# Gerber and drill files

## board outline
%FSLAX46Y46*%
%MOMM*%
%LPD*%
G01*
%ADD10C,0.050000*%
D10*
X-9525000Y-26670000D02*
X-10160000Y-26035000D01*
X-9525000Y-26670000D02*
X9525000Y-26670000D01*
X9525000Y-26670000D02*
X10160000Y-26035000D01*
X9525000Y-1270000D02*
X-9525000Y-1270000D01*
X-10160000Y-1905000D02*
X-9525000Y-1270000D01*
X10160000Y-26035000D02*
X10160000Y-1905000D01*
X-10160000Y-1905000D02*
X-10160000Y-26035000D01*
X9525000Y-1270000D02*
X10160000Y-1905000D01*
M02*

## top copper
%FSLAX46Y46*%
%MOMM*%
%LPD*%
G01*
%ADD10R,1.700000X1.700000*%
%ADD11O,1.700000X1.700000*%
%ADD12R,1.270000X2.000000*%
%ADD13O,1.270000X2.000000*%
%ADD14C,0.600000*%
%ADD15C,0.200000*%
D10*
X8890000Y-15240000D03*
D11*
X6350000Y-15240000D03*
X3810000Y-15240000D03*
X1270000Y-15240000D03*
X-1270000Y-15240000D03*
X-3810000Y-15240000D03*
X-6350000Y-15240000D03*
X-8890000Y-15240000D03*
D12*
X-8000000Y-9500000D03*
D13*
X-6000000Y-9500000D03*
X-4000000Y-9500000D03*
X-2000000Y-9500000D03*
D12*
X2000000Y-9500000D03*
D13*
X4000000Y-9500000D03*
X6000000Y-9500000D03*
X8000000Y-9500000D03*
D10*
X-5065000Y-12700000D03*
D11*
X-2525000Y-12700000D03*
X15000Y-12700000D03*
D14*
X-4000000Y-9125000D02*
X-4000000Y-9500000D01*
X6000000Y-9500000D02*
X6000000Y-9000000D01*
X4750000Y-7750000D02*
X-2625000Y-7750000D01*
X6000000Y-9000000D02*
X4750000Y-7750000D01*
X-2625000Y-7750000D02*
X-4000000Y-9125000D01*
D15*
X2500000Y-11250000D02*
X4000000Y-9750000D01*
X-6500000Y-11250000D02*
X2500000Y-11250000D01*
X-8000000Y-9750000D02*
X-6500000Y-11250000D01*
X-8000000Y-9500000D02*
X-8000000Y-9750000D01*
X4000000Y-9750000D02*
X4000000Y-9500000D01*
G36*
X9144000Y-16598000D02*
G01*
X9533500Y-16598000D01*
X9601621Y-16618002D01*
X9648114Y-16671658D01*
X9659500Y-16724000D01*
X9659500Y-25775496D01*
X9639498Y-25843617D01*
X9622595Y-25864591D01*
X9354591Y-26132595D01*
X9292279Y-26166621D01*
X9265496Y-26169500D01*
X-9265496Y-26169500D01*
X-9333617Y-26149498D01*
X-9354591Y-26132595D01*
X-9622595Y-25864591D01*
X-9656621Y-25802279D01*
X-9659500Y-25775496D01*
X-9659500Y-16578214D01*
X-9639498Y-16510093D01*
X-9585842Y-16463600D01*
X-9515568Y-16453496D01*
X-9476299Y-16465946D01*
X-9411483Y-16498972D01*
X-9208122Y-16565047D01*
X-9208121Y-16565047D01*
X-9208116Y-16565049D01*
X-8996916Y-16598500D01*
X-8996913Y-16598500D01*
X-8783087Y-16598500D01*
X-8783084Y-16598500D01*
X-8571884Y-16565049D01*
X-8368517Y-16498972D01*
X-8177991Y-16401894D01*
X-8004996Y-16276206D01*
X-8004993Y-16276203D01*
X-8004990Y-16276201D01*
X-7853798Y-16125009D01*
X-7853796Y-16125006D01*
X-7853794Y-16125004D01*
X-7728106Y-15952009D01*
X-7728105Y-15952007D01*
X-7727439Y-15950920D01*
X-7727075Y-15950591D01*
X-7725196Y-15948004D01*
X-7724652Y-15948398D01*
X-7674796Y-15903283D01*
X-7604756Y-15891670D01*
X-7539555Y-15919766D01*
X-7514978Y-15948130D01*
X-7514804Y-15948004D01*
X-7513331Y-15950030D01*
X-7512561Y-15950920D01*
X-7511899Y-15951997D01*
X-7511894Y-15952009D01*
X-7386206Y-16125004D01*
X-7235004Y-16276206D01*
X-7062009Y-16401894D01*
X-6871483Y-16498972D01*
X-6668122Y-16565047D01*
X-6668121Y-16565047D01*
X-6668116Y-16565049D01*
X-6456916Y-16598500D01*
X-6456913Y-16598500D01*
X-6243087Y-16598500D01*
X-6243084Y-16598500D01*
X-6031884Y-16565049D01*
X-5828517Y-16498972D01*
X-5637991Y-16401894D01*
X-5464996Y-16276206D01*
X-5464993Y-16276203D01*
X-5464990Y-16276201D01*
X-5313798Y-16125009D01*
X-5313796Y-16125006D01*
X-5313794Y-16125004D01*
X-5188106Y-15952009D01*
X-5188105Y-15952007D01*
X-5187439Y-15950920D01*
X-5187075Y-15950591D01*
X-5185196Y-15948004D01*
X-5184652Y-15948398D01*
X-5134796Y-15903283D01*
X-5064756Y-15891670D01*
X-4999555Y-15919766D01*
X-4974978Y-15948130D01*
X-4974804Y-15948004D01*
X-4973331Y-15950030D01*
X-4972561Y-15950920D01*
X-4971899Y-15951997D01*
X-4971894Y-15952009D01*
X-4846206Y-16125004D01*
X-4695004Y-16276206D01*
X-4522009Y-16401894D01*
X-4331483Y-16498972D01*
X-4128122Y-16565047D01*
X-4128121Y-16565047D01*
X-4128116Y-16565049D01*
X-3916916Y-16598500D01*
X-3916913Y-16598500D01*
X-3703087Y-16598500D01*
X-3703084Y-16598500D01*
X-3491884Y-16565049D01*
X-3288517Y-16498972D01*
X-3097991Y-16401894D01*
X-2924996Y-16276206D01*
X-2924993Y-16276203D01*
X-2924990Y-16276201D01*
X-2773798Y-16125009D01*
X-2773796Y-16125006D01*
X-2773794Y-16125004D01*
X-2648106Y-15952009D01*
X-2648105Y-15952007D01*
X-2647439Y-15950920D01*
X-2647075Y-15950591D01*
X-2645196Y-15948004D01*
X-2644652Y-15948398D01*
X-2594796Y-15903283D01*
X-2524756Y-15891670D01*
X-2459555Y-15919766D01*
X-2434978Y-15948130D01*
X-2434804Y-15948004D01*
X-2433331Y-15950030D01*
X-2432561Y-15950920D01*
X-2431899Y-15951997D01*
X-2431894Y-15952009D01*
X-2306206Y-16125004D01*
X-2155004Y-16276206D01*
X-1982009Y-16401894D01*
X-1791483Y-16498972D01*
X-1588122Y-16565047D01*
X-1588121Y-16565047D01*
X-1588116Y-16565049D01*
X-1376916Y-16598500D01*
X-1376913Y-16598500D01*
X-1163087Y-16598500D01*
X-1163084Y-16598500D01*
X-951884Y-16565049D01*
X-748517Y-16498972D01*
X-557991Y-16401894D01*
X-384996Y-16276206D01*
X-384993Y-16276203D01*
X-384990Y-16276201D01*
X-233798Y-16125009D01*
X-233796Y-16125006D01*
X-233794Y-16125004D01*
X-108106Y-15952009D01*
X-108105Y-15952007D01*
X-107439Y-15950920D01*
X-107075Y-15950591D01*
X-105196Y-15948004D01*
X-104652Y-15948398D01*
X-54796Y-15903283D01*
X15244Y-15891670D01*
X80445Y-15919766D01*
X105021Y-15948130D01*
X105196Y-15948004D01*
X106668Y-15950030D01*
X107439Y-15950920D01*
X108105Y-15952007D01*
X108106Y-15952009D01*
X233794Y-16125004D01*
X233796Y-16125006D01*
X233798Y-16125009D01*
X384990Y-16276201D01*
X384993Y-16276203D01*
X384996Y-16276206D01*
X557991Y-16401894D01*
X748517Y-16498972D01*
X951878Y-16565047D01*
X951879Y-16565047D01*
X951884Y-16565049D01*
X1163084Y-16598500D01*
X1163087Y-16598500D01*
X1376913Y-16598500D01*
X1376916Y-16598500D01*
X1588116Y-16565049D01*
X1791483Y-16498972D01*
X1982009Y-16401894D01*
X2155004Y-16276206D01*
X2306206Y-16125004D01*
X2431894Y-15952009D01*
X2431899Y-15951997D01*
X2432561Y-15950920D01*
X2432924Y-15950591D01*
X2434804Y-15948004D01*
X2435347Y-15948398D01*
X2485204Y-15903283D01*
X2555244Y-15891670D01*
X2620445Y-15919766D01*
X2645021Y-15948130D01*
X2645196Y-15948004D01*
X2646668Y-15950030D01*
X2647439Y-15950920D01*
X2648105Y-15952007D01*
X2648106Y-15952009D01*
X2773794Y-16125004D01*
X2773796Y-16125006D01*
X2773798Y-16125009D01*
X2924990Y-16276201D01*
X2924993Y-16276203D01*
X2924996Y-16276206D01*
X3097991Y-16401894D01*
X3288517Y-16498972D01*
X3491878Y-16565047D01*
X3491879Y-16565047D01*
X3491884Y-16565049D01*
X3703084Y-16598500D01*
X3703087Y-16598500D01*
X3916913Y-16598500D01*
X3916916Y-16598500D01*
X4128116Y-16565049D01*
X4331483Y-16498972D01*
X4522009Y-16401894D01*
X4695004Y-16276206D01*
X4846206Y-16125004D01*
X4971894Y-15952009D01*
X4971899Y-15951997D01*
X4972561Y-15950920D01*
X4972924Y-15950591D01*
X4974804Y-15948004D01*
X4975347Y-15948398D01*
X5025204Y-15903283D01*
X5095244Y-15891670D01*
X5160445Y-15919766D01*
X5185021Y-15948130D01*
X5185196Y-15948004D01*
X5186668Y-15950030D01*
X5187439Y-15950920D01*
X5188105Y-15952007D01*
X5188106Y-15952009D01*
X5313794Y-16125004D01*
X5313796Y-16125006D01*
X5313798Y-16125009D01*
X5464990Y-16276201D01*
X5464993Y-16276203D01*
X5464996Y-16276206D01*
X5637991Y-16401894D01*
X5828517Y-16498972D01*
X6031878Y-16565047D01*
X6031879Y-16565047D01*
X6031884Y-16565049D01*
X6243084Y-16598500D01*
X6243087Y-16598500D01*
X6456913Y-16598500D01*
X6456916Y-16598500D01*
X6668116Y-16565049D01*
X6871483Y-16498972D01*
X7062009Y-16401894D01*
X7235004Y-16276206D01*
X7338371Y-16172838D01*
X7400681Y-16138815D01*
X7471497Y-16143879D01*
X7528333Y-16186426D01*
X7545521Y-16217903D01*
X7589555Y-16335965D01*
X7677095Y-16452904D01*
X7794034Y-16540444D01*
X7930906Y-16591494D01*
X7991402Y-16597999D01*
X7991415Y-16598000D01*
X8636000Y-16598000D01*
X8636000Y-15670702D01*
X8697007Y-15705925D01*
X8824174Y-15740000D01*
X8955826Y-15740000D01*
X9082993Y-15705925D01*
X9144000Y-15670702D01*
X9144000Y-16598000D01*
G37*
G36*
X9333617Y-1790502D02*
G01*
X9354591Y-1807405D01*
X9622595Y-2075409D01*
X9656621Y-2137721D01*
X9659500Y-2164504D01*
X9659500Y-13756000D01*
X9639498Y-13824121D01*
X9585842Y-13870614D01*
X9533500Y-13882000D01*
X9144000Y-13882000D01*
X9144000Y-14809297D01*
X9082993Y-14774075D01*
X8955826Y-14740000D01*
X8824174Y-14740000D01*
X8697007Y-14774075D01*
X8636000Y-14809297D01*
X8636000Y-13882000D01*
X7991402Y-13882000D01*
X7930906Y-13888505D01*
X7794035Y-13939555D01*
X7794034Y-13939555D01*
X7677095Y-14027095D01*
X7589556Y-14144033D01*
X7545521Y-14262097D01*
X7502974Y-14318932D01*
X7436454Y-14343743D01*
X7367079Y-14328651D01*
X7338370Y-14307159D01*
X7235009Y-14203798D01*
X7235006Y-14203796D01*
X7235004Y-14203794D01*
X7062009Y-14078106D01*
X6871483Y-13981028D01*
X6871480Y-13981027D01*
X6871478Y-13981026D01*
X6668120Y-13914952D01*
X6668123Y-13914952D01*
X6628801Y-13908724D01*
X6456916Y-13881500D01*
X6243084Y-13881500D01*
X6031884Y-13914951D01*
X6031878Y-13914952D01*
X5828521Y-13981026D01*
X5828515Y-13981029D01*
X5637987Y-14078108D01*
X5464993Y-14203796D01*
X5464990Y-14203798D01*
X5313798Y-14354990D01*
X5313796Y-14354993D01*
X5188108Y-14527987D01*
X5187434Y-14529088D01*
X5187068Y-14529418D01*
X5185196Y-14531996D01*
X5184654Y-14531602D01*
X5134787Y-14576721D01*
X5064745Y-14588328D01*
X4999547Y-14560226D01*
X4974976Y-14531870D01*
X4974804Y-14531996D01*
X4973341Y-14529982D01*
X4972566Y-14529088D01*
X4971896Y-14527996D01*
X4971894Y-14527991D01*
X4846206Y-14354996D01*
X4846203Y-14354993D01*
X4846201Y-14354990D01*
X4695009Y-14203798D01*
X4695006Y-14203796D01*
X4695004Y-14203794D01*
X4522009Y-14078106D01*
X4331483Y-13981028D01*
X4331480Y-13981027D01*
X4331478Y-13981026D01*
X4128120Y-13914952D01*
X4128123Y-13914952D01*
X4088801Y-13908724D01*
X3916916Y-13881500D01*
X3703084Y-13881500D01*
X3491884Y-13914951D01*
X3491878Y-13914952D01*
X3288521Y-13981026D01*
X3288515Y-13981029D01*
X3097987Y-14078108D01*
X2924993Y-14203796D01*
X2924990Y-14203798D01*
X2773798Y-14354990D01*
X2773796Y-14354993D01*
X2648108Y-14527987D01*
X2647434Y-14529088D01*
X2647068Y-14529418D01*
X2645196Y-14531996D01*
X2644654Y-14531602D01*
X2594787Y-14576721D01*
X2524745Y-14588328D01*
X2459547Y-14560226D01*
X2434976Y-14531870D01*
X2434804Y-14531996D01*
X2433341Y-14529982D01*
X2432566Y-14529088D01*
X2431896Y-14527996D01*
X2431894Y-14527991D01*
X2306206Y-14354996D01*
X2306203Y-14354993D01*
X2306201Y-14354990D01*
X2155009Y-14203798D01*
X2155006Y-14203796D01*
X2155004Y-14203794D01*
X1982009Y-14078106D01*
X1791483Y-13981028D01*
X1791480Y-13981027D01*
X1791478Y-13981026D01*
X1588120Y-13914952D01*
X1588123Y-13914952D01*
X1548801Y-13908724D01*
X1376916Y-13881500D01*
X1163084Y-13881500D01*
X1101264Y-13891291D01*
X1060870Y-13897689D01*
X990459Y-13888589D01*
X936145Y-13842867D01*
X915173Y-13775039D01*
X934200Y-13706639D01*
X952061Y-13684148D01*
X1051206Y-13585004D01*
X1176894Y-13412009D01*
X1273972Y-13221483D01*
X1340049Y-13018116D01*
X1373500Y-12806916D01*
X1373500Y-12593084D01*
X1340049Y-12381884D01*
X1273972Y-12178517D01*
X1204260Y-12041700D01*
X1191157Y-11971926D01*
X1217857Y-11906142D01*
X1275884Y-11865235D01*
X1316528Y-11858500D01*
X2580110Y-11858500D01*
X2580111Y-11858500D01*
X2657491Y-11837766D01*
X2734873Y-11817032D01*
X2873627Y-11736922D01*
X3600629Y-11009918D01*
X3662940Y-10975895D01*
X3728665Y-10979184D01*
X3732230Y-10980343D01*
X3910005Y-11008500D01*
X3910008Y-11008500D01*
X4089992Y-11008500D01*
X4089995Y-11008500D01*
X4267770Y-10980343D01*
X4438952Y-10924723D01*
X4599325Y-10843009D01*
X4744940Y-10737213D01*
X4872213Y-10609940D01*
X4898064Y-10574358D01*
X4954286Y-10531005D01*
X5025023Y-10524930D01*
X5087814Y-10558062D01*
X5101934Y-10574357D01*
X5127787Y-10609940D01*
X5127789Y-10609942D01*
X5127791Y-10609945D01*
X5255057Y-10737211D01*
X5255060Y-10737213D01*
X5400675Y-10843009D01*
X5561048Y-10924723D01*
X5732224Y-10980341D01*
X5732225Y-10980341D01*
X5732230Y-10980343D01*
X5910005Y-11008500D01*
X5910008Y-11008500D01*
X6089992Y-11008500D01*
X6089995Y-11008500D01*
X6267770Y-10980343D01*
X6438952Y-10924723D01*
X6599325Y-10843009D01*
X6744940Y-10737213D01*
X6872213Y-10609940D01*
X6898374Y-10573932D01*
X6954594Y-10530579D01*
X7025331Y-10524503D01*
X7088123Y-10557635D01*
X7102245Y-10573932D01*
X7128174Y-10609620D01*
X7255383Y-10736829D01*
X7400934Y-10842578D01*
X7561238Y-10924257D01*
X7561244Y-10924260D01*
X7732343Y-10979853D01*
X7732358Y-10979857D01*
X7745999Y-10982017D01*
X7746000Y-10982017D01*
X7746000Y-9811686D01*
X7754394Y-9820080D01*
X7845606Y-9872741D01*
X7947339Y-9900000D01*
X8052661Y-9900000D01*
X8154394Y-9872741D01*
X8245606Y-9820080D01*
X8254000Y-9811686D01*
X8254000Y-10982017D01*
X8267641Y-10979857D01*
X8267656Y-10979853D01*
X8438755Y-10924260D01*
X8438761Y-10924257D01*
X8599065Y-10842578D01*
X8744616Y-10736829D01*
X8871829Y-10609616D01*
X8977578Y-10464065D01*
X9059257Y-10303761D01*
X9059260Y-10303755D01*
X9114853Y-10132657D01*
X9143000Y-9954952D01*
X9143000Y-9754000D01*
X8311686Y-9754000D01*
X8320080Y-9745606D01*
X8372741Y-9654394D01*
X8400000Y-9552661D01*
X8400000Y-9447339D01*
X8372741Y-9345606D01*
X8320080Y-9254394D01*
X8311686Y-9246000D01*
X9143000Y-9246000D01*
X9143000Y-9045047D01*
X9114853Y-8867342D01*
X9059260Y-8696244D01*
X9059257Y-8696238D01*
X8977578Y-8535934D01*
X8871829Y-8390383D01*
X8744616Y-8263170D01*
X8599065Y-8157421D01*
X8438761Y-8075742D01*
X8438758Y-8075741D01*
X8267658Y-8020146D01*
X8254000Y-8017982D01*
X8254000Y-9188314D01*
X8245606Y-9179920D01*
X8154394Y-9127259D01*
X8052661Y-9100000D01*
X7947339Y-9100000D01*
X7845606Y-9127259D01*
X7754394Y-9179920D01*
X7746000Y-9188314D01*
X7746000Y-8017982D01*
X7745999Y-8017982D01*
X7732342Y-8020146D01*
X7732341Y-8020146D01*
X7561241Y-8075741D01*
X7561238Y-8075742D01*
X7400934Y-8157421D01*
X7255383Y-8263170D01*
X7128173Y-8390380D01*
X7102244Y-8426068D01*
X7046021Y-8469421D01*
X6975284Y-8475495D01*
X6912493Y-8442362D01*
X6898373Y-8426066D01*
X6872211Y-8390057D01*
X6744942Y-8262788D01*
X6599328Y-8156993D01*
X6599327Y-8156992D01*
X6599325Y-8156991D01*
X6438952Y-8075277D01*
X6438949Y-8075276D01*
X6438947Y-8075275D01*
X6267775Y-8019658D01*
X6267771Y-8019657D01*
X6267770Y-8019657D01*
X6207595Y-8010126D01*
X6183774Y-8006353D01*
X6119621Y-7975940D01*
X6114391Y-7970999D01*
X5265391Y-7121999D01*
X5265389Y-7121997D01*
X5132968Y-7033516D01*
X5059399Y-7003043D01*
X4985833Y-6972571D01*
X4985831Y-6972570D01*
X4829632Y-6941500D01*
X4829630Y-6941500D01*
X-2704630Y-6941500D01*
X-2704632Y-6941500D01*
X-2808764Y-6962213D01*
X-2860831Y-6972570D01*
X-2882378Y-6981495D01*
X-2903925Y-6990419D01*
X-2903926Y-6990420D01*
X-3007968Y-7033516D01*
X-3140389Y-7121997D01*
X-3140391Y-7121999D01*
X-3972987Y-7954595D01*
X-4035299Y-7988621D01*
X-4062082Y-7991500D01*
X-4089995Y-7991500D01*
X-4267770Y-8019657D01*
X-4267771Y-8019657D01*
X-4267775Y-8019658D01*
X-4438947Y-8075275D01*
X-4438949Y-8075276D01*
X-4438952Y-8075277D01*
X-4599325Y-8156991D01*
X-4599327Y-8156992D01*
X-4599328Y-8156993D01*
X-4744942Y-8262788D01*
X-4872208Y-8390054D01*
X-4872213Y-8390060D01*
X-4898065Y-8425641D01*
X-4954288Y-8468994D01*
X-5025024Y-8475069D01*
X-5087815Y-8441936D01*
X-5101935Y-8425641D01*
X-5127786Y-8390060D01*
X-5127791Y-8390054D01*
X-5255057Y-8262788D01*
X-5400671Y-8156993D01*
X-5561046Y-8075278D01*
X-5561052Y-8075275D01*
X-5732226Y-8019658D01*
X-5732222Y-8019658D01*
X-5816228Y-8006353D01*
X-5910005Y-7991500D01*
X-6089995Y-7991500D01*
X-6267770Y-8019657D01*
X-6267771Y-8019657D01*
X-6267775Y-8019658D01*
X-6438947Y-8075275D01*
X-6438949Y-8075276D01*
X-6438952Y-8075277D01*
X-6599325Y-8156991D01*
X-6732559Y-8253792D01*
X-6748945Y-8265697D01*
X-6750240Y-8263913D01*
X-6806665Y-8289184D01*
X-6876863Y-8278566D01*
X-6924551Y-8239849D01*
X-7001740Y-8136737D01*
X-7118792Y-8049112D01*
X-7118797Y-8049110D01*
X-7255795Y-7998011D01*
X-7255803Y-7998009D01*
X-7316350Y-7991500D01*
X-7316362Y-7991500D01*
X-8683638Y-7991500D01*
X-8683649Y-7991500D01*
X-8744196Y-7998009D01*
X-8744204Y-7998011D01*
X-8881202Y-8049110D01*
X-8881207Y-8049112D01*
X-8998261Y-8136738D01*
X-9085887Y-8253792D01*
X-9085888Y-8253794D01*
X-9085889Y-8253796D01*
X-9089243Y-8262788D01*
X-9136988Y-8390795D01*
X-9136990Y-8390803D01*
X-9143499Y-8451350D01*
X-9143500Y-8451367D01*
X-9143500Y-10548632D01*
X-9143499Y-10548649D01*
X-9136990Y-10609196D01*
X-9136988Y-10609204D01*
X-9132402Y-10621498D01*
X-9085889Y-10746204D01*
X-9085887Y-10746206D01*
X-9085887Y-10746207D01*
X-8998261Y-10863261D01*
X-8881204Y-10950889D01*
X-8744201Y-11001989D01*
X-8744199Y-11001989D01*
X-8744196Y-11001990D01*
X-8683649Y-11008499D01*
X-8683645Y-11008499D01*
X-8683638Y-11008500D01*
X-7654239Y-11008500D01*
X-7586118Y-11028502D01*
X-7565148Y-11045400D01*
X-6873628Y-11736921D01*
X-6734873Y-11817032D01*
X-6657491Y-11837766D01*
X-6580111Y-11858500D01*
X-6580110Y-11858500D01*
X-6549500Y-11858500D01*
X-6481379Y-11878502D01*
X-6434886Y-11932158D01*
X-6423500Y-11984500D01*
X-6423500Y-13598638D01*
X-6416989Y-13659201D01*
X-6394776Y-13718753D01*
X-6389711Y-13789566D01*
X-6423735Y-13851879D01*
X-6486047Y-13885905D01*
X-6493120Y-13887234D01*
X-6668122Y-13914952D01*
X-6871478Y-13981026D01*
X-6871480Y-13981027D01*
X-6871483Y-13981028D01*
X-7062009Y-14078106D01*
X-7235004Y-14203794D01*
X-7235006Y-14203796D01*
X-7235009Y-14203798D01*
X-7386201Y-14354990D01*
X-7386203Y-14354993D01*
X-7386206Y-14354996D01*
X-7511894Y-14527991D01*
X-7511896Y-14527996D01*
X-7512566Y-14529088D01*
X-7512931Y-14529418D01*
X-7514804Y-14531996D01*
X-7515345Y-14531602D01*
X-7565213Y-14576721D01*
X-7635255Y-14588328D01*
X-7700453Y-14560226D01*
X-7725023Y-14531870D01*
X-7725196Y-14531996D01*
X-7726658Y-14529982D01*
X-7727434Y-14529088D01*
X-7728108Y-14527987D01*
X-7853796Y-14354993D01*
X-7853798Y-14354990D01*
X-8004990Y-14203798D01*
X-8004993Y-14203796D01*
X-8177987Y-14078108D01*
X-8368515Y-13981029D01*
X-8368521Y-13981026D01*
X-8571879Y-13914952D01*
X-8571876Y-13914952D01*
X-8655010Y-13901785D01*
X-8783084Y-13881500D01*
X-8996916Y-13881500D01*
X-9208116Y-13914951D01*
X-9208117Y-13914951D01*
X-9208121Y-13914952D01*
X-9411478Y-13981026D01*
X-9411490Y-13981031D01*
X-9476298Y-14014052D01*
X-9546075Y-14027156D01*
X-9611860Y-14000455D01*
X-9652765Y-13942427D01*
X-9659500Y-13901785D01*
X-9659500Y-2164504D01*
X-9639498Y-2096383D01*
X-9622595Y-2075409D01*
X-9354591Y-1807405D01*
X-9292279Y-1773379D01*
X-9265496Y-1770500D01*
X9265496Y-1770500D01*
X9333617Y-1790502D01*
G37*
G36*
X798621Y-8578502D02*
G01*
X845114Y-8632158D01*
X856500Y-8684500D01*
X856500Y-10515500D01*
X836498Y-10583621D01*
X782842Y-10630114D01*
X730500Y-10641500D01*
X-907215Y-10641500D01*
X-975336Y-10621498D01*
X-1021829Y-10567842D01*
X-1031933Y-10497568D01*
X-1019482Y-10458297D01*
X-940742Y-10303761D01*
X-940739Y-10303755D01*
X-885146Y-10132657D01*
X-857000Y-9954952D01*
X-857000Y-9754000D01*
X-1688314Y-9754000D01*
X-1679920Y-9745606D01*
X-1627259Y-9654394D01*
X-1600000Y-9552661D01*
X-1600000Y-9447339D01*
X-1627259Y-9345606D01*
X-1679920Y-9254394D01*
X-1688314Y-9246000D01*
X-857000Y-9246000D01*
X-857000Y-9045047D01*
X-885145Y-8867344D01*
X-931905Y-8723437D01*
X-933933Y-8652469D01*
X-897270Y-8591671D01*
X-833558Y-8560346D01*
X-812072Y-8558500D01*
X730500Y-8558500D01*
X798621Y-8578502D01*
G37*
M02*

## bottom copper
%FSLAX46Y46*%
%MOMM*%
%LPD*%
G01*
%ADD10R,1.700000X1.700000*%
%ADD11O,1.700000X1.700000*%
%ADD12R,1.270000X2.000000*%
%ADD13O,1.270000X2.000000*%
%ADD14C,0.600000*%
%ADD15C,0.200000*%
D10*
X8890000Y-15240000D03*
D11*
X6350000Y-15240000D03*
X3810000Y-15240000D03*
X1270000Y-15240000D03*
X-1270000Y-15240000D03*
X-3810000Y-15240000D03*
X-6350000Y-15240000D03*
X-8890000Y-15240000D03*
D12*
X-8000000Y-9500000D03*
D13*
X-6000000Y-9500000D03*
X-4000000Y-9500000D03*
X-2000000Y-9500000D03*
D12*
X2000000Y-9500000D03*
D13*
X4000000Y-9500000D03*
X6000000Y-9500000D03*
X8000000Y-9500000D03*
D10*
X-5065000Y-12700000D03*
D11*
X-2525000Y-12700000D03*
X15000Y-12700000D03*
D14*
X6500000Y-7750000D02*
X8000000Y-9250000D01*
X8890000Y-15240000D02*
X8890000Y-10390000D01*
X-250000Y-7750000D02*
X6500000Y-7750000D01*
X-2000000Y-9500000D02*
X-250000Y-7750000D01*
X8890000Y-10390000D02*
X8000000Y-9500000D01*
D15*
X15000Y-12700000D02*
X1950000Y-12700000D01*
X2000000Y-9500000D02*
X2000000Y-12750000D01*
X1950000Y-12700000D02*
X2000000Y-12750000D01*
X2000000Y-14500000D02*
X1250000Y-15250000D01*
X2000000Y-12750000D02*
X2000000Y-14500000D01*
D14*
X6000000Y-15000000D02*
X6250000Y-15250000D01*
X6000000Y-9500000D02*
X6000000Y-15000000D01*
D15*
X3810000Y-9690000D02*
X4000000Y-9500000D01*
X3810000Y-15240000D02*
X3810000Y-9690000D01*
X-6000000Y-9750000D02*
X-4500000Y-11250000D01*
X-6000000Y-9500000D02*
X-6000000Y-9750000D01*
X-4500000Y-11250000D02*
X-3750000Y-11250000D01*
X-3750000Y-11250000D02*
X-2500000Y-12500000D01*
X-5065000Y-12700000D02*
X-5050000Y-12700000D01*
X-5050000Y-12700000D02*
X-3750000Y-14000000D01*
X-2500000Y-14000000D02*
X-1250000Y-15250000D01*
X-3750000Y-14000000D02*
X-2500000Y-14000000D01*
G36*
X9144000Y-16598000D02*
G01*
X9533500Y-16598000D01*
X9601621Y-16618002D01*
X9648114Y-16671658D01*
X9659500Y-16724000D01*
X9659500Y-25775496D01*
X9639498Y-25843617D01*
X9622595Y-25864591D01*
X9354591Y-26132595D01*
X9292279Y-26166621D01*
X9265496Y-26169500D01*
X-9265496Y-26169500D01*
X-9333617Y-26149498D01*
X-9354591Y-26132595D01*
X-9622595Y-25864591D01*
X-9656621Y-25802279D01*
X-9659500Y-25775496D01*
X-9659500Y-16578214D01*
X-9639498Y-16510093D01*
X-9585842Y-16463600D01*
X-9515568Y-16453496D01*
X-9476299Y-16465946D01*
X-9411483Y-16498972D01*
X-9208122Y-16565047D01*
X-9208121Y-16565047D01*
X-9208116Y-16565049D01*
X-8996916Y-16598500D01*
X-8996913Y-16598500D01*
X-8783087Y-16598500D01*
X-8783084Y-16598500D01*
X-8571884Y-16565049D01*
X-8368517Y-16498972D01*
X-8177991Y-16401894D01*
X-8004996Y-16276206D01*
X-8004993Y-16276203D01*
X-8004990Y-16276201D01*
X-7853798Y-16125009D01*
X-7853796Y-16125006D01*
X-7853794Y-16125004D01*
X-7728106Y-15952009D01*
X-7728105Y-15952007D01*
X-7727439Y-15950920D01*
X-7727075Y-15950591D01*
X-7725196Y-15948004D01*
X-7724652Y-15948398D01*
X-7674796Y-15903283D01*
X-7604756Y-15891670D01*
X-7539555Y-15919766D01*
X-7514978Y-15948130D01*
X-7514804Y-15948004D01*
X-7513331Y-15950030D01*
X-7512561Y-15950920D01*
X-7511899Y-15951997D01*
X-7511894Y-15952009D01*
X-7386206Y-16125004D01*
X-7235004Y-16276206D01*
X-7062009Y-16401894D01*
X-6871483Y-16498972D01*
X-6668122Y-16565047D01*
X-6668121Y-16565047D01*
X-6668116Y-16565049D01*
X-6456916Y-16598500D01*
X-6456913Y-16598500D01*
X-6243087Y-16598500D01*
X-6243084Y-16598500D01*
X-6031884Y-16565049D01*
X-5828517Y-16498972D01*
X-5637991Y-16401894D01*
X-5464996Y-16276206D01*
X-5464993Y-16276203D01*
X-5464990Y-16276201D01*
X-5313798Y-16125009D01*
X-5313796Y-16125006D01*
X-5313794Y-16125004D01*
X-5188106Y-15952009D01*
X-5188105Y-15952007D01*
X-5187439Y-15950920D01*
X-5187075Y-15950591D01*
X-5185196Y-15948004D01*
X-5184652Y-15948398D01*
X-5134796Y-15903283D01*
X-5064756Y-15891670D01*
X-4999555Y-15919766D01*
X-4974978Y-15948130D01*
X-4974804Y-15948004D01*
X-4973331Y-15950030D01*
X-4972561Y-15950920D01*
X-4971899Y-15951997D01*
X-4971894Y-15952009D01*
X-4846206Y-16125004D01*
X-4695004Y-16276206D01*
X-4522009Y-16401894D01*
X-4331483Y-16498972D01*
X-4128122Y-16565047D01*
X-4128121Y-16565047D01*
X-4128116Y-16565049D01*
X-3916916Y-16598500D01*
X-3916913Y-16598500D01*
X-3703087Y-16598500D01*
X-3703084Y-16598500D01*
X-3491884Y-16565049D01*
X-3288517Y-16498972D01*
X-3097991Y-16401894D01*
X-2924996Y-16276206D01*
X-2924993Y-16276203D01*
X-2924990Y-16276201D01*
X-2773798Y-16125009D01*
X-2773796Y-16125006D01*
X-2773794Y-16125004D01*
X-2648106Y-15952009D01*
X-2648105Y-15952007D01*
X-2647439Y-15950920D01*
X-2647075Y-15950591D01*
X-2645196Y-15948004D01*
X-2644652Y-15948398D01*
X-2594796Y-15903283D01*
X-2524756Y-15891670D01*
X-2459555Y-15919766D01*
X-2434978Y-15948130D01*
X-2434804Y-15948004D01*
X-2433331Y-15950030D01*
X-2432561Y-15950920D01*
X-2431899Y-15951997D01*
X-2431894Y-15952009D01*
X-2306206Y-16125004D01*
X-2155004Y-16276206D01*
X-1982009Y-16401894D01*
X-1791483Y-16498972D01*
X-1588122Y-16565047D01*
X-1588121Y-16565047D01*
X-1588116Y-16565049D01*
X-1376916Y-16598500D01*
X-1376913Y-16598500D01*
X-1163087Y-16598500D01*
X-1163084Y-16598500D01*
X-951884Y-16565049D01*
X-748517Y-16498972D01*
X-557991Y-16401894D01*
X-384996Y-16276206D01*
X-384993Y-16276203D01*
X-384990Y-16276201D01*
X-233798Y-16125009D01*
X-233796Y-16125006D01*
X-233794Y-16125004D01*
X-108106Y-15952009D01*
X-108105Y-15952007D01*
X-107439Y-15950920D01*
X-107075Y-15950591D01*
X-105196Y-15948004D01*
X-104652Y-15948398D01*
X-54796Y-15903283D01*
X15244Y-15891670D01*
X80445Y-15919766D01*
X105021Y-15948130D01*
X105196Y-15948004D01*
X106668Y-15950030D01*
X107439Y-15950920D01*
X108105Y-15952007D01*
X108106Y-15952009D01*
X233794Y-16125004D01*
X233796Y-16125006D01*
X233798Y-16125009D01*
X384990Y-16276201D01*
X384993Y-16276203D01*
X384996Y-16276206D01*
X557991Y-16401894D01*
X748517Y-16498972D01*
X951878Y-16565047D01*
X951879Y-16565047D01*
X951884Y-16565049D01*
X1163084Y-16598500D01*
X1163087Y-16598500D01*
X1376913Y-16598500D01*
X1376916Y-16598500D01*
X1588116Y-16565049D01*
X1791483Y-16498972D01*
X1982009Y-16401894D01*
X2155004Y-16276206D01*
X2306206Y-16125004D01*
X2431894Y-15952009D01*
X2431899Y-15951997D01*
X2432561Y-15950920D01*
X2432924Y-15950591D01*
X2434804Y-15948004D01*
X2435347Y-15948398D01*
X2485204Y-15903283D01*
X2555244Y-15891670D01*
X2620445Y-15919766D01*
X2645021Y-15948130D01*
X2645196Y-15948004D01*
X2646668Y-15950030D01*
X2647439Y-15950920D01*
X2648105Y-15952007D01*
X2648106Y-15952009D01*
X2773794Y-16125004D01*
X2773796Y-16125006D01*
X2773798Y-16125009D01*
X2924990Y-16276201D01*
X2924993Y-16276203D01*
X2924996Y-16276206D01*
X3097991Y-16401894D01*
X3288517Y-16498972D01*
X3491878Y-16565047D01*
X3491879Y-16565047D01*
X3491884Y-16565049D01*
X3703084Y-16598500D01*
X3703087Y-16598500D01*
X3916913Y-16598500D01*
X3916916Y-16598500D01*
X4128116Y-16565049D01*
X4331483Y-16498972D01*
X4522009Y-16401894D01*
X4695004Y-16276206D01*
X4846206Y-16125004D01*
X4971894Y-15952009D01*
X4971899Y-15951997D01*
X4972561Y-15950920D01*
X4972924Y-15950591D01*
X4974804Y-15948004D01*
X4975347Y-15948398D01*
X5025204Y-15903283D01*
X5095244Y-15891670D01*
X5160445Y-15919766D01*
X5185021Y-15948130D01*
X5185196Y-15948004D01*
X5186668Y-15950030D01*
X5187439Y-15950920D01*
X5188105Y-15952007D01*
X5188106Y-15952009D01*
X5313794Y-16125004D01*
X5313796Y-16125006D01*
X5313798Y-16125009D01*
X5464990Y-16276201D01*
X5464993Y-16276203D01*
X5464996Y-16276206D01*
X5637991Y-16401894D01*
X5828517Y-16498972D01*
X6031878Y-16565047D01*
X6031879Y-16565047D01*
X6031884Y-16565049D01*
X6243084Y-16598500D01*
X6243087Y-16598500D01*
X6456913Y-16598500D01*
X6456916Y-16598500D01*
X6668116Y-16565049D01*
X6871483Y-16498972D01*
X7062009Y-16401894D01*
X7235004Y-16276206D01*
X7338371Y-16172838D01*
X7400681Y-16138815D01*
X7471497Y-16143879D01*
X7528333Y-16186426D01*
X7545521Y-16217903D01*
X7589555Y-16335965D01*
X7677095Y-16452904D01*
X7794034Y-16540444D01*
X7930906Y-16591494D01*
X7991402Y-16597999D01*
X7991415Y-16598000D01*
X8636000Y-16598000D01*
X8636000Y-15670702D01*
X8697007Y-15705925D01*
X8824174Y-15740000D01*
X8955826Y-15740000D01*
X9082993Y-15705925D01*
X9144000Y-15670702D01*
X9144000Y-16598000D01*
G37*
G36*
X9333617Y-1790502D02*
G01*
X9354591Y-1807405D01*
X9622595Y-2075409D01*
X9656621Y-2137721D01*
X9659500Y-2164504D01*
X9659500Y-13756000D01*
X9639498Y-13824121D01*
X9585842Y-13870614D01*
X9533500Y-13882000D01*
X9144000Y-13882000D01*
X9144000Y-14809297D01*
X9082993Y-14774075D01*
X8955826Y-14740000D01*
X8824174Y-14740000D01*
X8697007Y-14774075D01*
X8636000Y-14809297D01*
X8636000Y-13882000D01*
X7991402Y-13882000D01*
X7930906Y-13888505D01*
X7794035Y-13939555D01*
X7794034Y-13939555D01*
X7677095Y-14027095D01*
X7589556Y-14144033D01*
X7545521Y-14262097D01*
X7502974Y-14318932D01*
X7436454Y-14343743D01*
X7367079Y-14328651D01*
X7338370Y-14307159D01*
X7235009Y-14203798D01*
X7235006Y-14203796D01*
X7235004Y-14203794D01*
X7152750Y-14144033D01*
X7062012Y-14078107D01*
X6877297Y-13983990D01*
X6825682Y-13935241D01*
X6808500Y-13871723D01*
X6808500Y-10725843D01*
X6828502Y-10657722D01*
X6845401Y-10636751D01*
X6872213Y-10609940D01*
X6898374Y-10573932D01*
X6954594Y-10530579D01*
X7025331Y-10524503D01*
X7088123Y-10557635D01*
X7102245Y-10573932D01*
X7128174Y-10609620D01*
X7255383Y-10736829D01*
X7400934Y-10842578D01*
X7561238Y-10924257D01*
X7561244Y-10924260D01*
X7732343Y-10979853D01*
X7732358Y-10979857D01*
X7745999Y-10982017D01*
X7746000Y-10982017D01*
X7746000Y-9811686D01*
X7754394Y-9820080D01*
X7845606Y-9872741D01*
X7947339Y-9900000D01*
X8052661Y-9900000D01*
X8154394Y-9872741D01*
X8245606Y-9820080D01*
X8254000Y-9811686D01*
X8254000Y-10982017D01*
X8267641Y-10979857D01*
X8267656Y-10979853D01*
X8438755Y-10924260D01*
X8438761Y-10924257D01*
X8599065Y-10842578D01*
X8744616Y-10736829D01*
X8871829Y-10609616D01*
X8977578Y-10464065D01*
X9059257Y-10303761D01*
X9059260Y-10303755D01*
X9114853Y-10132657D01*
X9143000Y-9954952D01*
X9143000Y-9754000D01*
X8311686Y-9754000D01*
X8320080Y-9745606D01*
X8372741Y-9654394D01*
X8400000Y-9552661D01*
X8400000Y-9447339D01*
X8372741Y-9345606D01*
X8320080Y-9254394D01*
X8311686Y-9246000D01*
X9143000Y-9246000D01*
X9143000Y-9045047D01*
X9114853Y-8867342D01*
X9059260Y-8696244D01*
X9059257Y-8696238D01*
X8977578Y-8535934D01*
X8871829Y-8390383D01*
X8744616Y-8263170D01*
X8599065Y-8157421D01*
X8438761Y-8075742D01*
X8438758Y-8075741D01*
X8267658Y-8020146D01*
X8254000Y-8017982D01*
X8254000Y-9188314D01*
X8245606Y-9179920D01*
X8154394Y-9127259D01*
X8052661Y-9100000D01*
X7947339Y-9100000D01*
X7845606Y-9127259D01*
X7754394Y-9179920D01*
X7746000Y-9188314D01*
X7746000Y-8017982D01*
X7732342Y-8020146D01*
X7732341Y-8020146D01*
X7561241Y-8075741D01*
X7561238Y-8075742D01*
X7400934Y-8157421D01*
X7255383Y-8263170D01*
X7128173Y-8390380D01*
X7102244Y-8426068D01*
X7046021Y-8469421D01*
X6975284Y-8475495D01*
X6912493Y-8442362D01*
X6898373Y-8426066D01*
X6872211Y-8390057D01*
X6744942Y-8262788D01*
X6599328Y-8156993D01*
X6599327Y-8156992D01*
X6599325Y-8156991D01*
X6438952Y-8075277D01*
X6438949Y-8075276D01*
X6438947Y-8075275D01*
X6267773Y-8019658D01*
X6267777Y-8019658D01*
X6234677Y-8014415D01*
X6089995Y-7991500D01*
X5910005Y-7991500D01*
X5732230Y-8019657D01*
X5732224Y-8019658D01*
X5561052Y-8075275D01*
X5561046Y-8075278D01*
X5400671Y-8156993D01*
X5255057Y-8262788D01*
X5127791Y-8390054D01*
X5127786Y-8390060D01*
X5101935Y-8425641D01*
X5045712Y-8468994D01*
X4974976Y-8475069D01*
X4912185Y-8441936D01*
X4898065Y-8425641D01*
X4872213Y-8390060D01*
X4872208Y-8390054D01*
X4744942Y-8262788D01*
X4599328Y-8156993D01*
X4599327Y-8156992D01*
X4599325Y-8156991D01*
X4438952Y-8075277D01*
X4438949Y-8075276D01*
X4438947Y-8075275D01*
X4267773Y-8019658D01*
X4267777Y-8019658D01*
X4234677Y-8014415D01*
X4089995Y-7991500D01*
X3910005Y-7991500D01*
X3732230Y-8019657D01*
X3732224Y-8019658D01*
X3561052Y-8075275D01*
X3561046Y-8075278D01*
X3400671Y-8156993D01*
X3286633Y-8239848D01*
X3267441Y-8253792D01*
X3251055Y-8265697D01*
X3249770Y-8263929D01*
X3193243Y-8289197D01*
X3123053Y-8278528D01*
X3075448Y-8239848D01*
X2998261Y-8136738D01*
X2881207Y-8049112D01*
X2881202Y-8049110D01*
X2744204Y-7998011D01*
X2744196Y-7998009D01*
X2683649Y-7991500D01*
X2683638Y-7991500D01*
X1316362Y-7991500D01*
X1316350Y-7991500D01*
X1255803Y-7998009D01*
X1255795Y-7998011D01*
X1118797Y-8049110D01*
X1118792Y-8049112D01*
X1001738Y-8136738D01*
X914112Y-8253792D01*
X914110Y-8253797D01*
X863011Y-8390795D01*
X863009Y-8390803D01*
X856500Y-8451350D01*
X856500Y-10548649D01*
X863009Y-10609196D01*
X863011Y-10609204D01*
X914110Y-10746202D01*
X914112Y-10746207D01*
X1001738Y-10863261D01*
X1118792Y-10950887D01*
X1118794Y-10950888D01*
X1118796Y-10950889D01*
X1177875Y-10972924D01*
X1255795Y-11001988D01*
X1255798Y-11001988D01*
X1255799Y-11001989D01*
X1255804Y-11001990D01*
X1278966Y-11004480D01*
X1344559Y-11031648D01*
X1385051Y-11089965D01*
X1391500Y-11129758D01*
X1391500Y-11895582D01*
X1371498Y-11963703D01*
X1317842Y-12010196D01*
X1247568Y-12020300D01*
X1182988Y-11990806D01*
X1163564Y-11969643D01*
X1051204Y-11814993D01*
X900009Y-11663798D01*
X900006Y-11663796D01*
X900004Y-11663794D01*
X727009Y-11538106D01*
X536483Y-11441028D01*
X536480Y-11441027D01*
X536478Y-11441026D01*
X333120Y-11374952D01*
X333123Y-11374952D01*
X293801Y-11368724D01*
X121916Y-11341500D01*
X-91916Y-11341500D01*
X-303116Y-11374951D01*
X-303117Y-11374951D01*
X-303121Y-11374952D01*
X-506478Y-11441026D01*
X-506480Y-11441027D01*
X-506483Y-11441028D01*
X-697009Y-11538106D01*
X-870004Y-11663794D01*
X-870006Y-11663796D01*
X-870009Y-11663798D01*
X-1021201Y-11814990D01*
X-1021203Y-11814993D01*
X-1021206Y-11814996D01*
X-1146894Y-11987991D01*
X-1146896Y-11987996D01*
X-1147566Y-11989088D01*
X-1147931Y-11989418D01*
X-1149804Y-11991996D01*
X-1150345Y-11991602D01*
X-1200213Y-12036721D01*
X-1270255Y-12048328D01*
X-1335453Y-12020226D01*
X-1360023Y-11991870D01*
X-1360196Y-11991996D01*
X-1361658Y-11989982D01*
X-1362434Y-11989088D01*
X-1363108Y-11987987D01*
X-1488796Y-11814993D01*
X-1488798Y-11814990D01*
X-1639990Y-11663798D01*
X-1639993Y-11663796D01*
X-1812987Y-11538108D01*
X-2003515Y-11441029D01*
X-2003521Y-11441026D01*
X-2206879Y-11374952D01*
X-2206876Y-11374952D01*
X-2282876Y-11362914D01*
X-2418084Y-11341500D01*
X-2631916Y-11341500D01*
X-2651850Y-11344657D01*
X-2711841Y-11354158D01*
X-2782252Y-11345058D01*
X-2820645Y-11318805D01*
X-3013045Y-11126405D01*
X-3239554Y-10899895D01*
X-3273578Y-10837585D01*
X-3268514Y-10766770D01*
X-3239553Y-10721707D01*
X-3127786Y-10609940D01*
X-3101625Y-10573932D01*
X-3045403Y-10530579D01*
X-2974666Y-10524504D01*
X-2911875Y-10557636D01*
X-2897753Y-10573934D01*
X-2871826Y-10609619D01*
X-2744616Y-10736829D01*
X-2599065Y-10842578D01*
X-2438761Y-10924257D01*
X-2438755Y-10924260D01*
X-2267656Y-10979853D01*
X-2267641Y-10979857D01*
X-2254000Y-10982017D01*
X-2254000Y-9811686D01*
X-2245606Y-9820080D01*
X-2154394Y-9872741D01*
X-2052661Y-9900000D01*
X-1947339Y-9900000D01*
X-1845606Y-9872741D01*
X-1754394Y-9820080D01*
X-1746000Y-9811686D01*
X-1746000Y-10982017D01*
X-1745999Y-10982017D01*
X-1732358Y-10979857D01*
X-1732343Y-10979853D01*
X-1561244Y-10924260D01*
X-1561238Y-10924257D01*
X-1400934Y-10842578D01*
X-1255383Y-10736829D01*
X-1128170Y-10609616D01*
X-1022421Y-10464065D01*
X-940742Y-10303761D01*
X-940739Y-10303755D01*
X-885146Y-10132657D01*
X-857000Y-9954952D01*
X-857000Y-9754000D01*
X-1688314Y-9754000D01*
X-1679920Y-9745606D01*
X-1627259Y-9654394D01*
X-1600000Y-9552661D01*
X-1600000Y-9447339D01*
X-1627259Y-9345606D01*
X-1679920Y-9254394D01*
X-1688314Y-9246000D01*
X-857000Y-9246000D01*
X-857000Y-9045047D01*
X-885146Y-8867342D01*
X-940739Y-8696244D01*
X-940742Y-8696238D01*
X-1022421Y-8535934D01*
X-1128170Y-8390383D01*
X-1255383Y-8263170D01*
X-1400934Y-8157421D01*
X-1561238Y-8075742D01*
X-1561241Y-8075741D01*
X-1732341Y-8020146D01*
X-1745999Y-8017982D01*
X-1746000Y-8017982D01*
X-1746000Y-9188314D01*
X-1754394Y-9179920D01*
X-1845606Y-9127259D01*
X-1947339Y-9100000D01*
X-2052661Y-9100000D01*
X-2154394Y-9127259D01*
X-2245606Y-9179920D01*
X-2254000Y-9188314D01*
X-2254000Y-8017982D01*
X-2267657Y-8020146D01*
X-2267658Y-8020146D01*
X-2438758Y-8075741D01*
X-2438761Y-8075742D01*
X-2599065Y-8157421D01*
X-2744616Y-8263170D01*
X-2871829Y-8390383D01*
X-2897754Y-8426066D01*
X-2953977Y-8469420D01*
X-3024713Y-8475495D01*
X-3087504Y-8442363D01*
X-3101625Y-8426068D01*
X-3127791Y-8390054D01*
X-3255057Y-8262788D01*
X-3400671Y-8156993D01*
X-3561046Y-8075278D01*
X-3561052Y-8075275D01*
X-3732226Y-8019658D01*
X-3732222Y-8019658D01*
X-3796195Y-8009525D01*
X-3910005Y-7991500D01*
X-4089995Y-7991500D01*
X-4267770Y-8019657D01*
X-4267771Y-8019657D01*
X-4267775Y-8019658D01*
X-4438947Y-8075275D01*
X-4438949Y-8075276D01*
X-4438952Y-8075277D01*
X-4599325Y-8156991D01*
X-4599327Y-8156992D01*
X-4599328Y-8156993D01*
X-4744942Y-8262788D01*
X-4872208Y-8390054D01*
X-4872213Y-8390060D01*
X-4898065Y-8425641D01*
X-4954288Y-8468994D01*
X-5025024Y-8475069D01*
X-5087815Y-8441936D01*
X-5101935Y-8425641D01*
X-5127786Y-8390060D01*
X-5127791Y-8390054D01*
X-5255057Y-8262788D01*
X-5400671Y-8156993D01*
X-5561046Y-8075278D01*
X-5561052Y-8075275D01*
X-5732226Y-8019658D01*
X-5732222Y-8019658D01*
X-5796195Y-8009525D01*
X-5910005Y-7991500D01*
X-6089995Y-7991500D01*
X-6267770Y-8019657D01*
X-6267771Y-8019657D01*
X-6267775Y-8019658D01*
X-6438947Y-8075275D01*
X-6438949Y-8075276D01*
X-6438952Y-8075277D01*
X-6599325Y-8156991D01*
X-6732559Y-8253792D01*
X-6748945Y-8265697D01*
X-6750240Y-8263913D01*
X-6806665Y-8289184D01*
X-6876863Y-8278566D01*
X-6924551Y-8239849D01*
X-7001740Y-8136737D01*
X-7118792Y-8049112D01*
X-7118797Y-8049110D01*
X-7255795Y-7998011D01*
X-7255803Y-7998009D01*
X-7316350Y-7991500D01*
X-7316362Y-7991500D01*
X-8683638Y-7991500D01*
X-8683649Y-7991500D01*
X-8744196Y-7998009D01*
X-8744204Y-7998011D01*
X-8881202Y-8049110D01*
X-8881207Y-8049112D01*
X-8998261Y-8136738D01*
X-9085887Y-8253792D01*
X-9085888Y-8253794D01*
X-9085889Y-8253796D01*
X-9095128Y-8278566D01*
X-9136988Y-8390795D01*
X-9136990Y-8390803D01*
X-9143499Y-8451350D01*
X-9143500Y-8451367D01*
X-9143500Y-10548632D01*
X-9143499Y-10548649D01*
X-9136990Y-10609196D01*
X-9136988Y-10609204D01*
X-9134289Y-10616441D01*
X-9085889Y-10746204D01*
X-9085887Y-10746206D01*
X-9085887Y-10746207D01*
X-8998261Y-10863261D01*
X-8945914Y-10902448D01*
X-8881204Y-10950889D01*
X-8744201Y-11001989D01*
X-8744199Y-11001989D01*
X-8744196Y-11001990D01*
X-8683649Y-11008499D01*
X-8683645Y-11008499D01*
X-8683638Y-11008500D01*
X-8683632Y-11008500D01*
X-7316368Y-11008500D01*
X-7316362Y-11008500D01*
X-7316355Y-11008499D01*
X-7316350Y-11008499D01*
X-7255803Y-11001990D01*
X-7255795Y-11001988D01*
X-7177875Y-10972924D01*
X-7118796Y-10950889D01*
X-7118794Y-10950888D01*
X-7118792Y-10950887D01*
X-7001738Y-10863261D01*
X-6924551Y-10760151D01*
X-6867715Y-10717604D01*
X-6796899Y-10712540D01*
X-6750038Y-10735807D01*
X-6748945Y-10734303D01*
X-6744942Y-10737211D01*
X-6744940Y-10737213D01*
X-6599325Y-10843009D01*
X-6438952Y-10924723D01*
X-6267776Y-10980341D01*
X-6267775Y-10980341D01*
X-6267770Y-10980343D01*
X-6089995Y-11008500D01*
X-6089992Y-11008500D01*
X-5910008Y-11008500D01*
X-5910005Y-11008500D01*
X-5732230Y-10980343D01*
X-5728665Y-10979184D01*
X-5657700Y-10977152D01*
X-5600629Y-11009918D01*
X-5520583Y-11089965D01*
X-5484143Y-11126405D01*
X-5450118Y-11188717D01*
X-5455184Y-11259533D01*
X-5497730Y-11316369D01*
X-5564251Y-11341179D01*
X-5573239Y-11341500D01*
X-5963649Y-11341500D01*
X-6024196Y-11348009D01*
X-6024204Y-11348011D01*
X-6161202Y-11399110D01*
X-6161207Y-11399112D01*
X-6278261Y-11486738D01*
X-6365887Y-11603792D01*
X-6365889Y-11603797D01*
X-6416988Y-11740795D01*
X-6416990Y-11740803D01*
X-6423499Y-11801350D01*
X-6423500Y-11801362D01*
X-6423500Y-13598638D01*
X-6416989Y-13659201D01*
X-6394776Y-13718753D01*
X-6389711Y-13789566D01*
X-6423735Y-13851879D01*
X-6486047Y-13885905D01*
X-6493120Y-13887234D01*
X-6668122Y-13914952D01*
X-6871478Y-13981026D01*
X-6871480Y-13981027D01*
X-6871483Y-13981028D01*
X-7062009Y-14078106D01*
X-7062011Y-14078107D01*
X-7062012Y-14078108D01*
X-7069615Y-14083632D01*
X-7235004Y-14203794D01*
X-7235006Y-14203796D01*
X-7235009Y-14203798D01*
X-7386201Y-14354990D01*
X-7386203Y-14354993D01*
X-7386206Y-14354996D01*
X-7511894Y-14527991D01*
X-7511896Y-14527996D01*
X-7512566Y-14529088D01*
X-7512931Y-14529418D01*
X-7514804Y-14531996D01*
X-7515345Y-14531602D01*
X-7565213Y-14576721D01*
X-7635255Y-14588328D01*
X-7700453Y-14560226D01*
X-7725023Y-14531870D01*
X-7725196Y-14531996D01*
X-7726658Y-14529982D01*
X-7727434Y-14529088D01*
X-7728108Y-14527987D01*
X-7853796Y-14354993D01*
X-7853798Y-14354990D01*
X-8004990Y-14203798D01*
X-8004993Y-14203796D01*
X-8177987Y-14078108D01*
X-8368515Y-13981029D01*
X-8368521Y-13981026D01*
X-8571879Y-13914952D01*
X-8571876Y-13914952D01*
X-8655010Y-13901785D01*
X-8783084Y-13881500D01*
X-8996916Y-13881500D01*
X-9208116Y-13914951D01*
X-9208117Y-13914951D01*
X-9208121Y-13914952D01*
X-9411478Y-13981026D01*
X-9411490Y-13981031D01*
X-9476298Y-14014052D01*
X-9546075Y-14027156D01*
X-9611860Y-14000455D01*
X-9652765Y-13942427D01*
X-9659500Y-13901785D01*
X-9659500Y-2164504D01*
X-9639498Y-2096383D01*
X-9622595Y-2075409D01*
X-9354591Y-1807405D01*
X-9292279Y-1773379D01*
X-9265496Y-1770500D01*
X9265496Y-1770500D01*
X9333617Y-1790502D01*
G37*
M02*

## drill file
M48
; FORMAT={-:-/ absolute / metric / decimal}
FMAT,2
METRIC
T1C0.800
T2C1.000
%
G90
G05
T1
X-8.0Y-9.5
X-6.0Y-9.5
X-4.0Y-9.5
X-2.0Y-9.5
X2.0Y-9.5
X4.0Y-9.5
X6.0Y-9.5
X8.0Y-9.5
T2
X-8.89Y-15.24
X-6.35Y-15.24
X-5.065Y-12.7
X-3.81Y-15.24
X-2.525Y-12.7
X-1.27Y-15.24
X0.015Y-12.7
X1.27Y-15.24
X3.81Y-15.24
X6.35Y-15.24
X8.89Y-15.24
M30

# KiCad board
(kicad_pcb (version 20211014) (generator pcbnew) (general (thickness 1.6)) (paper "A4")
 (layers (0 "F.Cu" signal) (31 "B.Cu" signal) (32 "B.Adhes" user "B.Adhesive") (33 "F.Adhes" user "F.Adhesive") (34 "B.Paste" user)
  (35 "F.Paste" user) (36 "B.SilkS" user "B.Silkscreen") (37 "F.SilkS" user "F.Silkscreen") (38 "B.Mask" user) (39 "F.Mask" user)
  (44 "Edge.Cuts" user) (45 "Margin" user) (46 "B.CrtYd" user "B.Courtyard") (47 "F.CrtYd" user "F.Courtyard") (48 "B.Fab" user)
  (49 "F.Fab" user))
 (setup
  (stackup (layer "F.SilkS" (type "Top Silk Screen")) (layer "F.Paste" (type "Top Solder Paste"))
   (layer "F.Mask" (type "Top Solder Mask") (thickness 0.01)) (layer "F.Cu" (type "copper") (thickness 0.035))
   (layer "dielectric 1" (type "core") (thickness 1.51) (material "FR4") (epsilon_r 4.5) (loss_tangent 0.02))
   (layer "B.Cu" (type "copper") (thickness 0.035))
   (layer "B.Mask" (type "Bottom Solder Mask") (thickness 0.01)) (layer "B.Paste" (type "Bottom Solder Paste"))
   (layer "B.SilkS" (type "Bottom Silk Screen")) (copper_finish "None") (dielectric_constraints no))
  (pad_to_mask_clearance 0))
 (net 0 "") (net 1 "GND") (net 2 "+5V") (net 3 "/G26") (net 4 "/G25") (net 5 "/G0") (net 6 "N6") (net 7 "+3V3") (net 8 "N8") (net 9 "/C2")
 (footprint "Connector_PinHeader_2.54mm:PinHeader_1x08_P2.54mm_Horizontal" (layer "F.Cu") (at 8.89 15.24 -90)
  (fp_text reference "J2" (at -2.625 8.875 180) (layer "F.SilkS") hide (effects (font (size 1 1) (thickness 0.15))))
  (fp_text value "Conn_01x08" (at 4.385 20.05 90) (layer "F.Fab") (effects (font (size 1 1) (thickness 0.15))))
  (pad "1" thru_hole rect locked (at 0 0 270) (size 1.7 1.7) (drill 1) (layers *.Cu *.Mask) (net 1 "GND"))
  (pad "2" thru_hole oval locked (at 0 2.54 270) (size 1.7 1.7) (drill 1) (layers *.Cu *.Mask) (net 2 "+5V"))
  (pad "3" thru_hole oval locked (at 0 5.08 270) (size 1.7 1.7) (drill 1) (layers *.Cu *.Mask) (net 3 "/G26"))
  (pad "4" thru_hole oval locked (at 0 7.62 270) (size 1.7 1.7) (drill 1) (layers *.Cu *.Mask) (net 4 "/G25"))
  (pad "5" thru_hole oval locked (at 0 10.16 270) (size 1.7 1.7) (drill 1) (layers *.Cu *.Mask) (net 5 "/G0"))
  (pad "6" thru_hole oval locked (at 0 12.7 270) (size 1.7 1.7) (drill 1) (layers *.Cu *.Mask) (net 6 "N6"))
  (pad "7" thru_hole oval locked (at 0 15.24 270) (size 1.7 1.7) (drill 1) (layers *.Cu *.Mask) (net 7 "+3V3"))
  (pad "8" thru_hole oval locked (at 0 17.78 270) (size 1.7 1.7) (drill 1) (layers *.Cu *.Mask) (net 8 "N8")))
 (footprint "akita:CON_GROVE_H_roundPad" (layer "F.Cu") (at -5 9.5)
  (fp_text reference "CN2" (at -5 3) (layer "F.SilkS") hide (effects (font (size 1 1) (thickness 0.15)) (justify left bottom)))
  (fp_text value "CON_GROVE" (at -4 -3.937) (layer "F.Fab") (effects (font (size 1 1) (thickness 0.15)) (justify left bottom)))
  (pad "1" thru_hole rect (at -3 0) (size 1.27 2) (drill 0.8) (layers *.Cu *.Mask) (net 3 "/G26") (solder_mask_margin 0.1016))
  (pad "2" thru_hole oval (at -1 0) (size 1.27 2) (drill 0.8) (layers *.Cu *.Mask) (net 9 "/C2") (solder_mask_margin 0.1016))
  (pad "3" thru_hole oval (at 1 0) (size 1.27 2) (drill 0.8) (layers *.Cu *.Mask) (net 2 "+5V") (solder_mask_margin 0.1016))
  (pad "4" thru_hole oval (at 3 0) (size 1.27 2) (drill 0.8) (layers *.Cu *.Mask) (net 1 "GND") (solder_mask_margin 0.1016)))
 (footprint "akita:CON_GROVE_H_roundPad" (layer "F.Cu") (at 5 9.5)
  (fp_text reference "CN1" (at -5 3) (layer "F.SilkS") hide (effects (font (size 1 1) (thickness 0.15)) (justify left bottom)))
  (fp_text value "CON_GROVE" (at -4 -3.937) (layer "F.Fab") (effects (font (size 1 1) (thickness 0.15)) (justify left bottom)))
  (pad "1" thru_hole rect (at -3 0) (size 1.27 2) (drill 0.8) (layers *.Cu *.Mask) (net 4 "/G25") (solder_mask_margin 0.1016))
  (pad "2" thru_hole oval (at -1 0) (size 1.27 2) (drill 0.8) (layers *.Cu *.Mask) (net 3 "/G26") (solder_mask_margin 0.1016))
  (pad "3" thru_hole oval (at 1 0) (size 1.27 2) (drill 0.8) (layers *.Cu *.Mask) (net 2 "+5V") (solder_mask_margin 0.1016))
  (pad "4" thru_hole oval (at 3 0) (size 1.27 2) (drill 0.8) (layers *.Cu *.Mask) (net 1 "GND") (solder_mask_margin 0.1016)))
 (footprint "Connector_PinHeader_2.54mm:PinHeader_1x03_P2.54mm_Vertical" (layer "F.Cu") (at -5.065 12.7 90)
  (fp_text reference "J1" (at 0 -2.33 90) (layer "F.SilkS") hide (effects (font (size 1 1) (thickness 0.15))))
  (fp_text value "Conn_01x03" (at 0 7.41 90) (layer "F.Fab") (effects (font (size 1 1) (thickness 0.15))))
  (pad "1" thru_hole rect locked (at 0 0 90) (size 1.7 1.7) (drill 1) (layers *.Cu *.Mask) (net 5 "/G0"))
  (pad "2" thru_hole oval locked (at 0 2.54 90) (size 1.7 1.7) (drill 1) (layers *.Cu *.Mask) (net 9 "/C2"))
  (pad "3" thru_hole oval locked (at 0 5.08 90) (size 1.7 1.7) (drill 1) (layers *.Cu *.Mask) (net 4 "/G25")))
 (gr_line (start -9.525 26.67) (end -10.16 26.035) (layer "Edge.Cuts") (width 0.05))
 (gr_line (start -9.525 26.67) (end 9.525 26.67) (layer "Edge.Cuts") (width 0.05))
 (gr_line (start 9.525 26.67) (end 10.16 26.035) (layer "Edge.Cuts") (width 0.05))
 (gr_line (start 9.525 1.27) (end -9.525 1.27) (layer "Edge.Cuts") (width 0.05))
 (gr_line (start -10.16 1.905) (end -9.525 1.27) (layer "Edge.Cuts") (width 0.05))
 (gr_line (start 10.16 26.035) (end 10.16 1.905) (layer "Edge.Cuts") (width 0.05))
 (gr_line (start -10.16 1.905) (end -10.16 26.035) (layer "Edge.Cuts") (width 0.05))
 (gr_line (start 9.525 1.27) (end 10.16 1.905) (layer "Edge.Cuts") (width 0.05))
 (segment (start 6.5 7.75) (end 8 9.25) (width 0.6) (layer "B.Cu") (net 1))
 (segment (start 8.89 15.24) (end 8.89 10.39) (width 0.6) (layer "B.Cu") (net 1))
 (segment (start -0.25 7.75) (end 6.5 7.75) (width 0.6) (layer "B.Cu") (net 1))
 (segment (start -2 9.5) (end -0.25 7.75) (width 0.6) (layer "B.Cu") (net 1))
 (segment (start 8.89 10.39) (end 8 9.5) (width 0.6) (layer "B.Cu") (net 1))
 (segment (start 0.015 12.7) (end 1.95 12.7) (width 0.2) (layer "B.Cu") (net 4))
 (segment (start 2 9.5) (end 2 12.75) (width 0.2) (layer "B.Cu") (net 4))
 (segment (start 1.95 12.7) (end 2 12.75) (width 0.2) (layer "B.Cu") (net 4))
 (segment (start 2 14.5) (end 1.25 15.25) (width 0.2) (layer "B.Cu") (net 4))
 (segment (start 2 12.75) (end 2 14.5) (width 0.2) (layer "B.Cu") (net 4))
 (segment (start -4 9.125) (end -4 9.5) (width 0.6) (layer "F.Cu") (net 2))
 (segment (start 6 9.5) (end 6 9) (width 0.6) (layer "F.Cu") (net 2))
 (segment (start 4.75 7.75) (end -2.625 7.75) (width 0.6) (layer "F.Cu") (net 2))
 (segment (start 6 9) (end 4.75 7.75) (width 0.6) (layer "F.Cu") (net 2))
 (segment (start -2.625 7.75) (end -4 9.125) (width 0.6) (layer "F.Cu") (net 2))
 (segment (start 6 15) (end 6.25 15.25) (width 0.6) (layer "B.Cu") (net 2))
 (segment (start 6 9.5) (end 6 15) (width 0.6) (layer "B.Cu") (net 2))
 (segment (start 2.5 11.25) (end 4 9.75) (width 0.2) (layer "F.Cu") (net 3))
 (segment (start -6.5 11.25) (end 2.5 11.25) (width 0.2) (layer "F.Cu") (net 3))
 (segment (start -8 9.75) (end -6.5 11.25) (width 0.2) (layer "F.Cu") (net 3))
 (segment (start -8 9.5) (end -8 9.75) (width 0.2) (layer "F.Cu") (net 3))
 (segment (start 4 9.75) (end 4 9.5) (width 0.2) (layer "F.Cu") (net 3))
 (segment (start 3.81 9.69) (end 4 9.5) (width 0.2) (layer "B.Cu") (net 3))
 (segment (start 3.81 15.24) (end 3.81 9.69) (width 0.2) (layer "B.Cu") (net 3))
 (segment (start -6 9.75) (end -4.5 11.25) (width 0.2) (layer "B.Cu") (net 9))
 (segment (start -6 9.5) (end -6 9.75) (width 0.2) (layer "B.Cu") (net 9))
 (segment (start -4.5 11.25) (end -3.75 11.25) (width 0.2) (layer "B.Cu") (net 9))
 (segment (start -3.75 11.25) (end -2.5 12.5) (width 0.2) (layer "B.Cu") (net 9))
 (segment (start -5.065 12.7) (end -5.05 12.7) (width 0.2) (layer "B.Cu") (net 5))
 (segment (start -5.05 12.7) (end -3.75 14) (width 0.2) (layer "B.Cu") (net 5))
 (segment (start -2.5 14) (end -1.25 15.25) (width 0.2) (layer "B.Cu") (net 5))
 (segment (start -3.75 14) (end -2.5 14) (width 0.2) (layer "B.Cu") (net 5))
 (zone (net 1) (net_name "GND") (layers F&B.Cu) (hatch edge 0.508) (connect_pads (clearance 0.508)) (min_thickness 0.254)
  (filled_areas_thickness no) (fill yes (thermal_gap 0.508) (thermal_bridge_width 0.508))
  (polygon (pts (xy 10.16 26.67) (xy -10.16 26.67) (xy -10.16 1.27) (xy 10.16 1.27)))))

